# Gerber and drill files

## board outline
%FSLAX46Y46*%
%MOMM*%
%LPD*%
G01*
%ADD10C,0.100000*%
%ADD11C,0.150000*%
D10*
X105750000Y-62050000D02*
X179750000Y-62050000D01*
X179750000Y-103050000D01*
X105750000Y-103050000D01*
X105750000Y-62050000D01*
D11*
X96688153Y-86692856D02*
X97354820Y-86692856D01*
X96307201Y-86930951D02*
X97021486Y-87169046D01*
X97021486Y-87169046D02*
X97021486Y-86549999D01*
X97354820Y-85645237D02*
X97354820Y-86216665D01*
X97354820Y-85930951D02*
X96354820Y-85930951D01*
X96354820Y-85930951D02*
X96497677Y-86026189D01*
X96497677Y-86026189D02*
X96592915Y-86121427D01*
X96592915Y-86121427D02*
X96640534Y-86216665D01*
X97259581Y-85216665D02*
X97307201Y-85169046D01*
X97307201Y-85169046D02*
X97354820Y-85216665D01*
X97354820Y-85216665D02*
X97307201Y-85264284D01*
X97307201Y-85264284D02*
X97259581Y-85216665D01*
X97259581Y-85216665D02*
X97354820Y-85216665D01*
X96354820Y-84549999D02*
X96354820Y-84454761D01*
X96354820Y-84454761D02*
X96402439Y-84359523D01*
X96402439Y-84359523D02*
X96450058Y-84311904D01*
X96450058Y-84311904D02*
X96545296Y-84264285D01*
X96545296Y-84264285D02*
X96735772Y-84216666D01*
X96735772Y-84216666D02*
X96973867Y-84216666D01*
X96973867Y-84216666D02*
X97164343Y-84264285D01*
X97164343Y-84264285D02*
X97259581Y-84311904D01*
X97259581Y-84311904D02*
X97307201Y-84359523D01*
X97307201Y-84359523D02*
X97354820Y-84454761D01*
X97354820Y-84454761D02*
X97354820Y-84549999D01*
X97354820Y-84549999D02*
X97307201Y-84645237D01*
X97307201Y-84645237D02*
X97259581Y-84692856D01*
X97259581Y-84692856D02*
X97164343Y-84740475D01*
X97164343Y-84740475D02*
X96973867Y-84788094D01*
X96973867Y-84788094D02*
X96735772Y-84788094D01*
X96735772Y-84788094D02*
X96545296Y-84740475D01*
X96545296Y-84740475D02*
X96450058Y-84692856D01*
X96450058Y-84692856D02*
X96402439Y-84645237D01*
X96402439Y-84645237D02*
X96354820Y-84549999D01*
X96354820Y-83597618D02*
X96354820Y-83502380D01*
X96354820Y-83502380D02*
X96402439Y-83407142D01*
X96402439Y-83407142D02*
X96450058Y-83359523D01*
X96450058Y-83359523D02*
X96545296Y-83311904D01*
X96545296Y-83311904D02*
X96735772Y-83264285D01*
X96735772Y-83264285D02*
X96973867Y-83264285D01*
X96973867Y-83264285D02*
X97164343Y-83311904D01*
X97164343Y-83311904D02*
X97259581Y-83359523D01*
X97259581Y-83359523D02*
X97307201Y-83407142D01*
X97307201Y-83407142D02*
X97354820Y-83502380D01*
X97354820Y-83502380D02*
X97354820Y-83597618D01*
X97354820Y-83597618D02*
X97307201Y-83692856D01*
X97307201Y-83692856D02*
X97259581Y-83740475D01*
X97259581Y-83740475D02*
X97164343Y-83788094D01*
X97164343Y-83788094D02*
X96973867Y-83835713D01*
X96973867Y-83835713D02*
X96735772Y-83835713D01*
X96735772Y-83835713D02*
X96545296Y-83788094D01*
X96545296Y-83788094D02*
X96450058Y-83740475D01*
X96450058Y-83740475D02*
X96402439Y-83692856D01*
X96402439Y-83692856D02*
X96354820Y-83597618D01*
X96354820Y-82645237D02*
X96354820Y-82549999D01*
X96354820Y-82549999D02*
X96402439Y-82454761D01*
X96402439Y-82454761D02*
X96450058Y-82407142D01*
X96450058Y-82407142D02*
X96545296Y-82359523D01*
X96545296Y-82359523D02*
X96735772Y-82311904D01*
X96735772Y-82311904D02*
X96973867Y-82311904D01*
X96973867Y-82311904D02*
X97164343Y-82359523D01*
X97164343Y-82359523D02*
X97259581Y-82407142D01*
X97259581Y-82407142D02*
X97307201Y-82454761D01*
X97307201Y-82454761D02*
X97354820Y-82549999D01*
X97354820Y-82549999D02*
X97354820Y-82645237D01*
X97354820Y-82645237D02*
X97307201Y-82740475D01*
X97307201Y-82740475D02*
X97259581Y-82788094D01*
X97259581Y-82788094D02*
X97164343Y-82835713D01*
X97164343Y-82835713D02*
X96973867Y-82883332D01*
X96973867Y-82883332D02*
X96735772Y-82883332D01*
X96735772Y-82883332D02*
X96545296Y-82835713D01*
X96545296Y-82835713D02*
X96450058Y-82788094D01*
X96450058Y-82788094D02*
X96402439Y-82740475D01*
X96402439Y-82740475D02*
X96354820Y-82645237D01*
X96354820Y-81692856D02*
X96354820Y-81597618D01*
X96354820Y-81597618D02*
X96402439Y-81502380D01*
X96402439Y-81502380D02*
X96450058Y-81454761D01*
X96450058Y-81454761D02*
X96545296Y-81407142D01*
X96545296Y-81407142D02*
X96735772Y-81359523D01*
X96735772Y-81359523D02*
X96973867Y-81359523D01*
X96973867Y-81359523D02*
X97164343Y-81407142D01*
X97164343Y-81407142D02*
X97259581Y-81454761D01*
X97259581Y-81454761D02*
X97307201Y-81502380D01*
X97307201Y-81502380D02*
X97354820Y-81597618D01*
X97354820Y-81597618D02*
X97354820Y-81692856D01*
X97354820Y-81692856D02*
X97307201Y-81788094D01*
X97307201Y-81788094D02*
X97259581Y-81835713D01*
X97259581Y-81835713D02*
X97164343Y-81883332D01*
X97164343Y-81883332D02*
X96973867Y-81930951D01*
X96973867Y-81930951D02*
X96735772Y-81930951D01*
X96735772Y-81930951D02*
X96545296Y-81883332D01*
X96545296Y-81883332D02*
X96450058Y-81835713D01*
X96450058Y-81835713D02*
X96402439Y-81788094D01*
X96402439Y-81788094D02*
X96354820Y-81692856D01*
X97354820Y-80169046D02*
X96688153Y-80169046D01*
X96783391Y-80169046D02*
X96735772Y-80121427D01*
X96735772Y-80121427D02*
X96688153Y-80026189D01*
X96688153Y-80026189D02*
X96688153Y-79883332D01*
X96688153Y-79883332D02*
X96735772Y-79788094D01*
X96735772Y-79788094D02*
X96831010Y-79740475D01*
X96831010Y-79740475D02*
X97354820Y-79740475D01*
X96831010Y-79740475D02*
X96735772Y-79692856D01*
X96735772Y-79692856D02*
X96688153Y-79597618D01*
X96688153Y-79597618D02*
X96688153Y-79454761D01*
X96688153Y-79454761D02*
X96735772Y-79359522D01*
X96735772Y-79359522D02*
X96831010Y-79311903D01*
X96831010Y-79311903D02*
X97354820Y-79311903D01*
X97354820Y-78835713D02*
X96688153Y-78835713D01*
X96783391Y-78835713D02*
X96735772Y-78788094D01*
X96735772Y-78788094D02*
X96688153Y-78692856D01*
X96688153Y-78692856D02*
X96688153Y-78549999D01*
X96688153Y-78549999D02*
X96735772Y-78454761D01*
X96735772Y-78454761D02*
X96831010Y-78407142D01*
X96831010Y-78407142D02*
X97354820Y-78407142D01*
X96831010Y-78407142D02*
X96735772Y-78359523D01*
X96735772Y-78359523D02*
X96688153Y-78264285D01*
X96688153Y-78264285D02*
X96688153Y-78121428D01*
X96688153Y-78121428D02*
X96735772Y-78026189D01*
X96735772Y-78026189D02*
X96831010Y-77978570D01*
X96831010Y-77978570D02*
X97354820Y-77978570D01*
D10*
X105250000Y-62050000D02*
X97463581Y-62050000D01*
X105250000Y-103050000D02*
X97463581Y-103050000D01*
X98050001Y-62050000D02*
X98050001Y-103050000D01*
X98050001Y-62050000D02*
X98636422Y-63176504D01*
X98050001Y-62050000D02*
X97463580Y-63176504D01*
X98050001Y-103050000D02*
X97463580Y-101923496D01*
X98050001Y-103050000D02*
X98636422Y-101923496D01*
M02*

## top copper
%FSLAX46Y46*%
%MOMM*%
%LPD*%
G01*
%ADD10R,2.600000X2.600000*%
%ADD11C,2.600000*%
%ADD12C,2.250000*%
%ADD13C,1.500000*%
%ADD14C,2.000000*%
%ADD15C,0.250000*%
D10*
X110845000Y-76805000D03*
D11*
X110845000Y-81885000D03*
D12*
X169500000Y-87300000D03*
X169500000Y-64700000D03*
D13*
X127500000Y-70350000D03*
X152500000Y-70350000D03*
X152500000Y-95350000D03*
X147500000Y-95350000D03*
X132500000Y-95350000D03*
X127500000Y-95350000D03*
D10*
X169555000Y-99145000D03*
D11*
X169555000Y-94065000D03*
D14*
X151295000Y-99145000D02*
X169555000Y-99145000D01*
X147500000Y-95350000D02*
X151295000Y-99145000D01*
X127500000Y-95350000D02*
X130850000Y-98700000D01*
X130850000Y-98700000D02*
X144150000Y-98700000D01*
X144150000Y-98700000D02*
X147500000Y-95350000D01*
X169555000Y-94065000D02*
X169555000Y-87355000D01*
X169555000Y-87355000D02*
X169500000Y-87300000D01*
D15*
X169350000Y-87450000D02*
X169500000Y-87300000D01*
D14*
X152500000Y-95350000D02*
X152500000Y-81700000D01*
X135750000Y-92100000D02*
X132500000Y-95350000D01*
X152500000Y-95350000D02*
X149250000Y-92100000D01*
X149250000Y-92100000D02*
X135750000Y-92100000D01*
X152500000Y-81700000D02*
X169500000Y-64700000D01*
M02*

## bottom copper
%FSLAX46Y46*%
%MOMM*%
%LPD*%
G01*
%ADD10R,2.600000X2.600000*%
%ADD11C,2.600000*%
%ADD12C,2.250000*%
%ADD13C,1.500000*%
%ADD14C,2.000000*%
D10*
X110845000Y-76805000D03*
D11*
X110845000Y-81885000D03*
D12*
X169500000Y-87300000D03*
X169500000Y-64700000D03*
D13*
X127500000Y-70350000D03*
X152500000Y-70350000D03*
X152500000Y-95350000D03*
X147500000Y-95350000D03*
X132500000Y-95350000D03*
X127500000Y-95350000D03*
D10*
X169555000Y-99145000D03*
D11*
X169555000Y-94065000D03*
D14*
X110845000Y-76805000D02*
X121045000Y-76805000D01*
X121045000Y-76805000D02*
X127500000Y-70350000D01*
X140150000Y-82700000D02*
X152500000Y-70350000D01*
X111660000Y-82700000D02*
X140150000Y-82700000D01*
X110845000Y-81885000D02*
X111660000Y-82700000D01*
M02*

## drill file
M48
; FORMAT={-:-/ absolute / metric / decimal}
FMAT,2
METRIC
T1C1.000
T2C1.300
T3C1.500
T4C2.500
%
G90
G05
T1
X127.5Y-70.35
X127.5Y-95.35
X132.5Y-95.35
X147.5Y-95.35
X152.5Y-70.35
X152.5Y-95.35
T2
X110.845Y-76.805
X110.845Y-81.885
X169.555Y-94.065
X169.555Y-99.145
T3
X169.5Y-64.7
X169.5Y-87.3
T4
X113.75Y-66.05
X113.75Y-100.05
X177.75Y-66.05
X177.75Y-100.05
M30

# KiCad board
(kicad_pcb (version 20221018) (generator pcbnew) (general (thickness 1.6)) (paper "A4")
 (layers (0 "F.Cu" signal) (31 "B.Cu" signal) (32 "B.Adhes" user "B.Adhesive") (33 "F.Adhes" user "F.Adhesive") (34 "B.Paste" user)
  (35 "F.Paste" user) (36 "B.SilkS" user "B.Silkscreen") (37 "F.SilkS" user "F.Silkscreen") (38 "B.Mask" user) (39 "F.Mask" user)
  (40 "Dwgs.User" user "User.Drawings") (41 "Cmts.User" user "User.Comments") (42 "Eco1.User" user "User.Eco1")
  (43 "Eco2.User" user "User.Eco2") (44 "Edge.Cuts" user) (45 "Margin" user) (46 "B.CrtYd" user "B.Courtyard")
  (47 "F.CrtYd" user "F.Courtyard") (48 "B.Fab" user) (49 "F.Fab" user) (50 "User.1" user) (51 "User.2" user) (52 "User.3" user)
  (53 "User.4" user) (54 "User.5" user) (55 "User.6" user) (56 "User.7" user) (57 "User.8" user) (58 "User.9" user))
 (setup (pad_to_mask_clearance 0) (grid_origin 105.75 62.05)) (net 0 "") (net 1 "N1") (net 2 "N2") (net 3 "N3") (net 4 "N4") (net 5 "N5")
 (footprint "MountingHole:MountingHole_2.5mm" (layer "F.Cu") (at 113.75 100.05)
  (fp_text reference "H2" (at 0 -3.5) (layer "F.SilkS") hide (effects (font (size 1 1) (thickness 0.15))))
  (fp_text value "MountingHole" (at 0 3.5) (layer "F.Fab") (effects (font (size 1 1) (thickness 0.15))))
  (pad "" np_thru_hole circle (at 0 0) (size 2.5 2.5) (drill 2.5) (layers "*.Cu" "*.Mask")))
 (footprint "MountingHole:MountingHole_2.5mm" (layer "F.Cu") (at 113.75 66.05)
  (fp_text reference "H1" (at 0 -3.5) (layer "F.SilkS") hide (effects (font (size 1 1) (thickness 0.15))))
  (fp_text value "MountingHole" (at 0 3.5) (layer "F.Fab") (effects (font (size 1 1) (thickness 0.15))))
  (pad "" np_thru_hole circle (at 0 0) (size 2.5 2.5) (drill 2.5) (layers "*.Cu" "*.Mask")))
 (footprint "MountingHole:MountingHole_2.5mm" (layer "F.Cu") (at 177.75 100.05)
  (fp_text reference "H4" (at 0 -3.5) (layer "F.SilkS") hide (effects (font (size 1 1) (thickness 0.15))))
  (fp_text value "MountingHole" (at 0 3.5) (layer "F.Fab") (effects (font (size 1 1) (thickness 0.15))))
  (pad "" np_thru_hole circle (at 0 0) (size 2.5 2.5) (drill 2.5) (layers "*.Cu" "*.Mask")))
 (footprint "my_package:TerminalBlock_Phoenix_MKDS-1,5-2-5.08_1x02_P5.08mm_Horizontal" (layer "F.Cu") (at 110.845 76.805 -90)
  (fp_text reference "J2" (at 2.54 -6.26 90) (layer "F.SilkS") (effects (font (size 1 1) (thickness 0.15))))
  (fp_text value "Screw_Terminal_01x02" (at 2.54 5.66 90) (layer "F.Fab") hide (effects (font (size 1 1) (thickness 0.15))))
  (pad "1" thru_hole rect (at 0 0 270) (size 2.6 2.6) (drill 1.3) (layers "*.Cu" "*.Mask") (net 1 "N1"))
  (pad "2" thru_hole circle (at 5.08 0 270) (size 2.6 2.6) (drill 1.3) (layers "*.Cu" "*.Mask") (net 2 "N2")))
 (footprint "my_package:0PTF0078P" (layer "F.Cu") (at 169.5 76 90)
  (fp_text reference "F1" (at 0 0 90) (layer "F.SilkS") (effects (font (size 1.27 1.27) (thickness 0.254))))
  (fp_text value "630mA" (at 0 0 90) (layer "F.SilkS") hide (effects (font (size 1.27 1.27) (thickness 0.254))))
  (pad "1" thru_hole circle (at -11.3 0 90) (size 2.25 2.25) (drill 1.5) (layers "*.Cu" "*.Mask") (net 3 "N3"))
  (pad "2" thru_hole circle (at 11.3 0 90) (size 2.25 2.25) (drill 1.5) (layers "*.Cu" "*.Mask") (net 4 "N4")))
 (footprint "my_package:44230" (layer "F.Cu") (at 127.5 70.35)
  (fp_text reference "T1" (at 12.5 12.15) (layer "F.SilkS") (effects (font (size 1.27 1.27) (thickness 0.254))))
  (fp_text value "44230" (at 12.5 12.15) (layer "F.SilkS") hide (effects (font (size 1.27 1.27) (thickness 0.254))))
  (pad "1" thru_hole circle (at 0 0) (size 1.5 1.5) (drill 1) (layers "*.Cu" "*.Mask") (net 1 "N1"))
  (pad "5" thru_hole circle (at 25 0) (size 1.5 1.5) (drill 1) (layers "*.Cu" "*.Mask") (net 2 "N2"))
  (pad "6" thru_hole circle (at 25 25) (size 1.5 1.5) (drill 1) (layers "*.Cu" "*.Mask") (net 4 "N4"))
  (pad "7" thru_hole circle (at 20 25) (size 1.5 1.5) (drill 1) (layers "*.Cu" "*.Mask") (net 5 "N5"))
  (pad "9" thru_hole circle (at 5 25) (size 1.5 1.5) (drill 1) (layers "*.Cu" "*.Mask") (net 4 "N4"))
  (pad "10" thru_hole circle (at 0 25) (size 1.5 1.5) (drill 1) (layers "*.Cu" "*.Mask") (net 5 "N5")))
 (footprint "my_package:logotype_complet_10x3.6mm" (layer "F.Cu") (at 111.4 70.95)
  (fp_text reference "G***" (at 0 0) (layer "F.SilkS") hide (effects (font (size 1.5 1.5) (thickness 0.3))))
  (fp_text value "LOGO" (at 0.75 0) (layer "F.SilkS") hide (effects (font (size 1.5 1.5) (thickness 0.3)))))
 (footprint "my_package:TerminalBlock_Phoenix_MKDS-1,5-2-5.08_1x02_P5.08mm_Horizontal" (layer "F.Cu") (at 169.555 99.145 90)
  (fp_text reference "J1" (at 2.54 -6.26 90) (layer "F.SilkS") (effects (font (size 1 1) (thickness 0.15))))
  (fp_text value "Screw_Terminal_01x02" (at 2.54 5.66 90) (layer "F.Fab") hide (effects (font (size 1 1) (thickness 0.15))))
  (pad "1" thru_hole rect (at 0 0 90) (size 2.6 2.6) (drill 1.3) (layers "*.Cu" "*.Mask") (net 5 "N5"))
  (pad "2" thru_hole circle (at 5.08 0 90) (size 2.6 2.6) (drill 1.3) (layers "*.Cu" "*.Mask") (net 3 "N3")))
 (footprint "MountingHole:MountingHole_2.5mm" (layer "F.Cu") (at 177.75 66.05)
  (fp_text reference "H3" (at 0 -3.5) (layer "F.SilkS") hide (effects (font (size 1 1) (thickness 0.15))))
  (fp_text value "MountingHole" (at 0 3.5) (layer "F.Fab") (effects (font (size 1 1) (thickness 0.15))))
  (pad "" np_thru_hole circle (at 0 0) (size 2.5 2.5) (drill 2.5) (layers "*.Cu" "*.Mask")))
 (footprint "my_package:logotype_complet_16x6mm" (layer "B.Cu") (at 142.75 67.05 180)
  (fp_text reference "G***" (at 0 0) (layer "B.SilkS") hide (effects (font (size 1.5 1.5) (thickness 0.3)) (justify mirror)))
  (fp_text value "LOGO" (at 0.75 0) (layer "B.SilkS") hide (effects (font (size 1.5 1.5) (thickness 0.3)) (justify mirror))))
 (gr_rect locked (start 105.75 62.05) (end 179.75 103.05) (stroke (width 0.1) (type default)) (fill none) (layer "Edge.Cuts"))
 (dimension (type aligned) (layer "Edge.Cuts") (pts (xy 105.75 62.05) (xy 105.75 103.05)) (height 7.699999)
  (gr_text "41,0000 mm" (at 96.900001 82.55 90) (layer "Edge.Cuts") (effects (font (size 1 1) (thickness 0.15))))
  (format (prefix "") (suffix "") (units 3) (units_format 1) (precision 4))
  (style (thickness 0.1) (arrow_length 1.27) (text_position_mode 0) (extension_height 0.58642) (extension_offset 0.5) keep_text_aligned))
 (segment (start 151.295 99.145) (end 169.555 99.145) (width 2) (layer "F.Cu") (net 5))
 (segment (start 147.5 95.35) (end 151.295 99.145) (width 2) (layer "F.Cu") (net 5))
 (segment (start 127.5 95.35) (end 130.85 98.7) (width 2) (layer "F.Cu") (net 5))
 (segment (start 130.85 98.7) (end 144.15 98.7) (width 2) (layer "F.Cu") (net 5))
 (segment (start 144.15 98.7) (end 147.5 95.35) (width 2) (layer "F.Cu") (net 5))
 (segment (start 169.555 94.065) (end 169.555 87.355) (width 2) (layer "F.Cu") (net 3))
 (segment (start 169.555 87.355) (end 169.5 87.3) (width 2) (layer "F.Cu") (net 3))
 (segment (start 169.35 87.45) (end 169.5 87.3) (width 0.25) (layer "F.Cu") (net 3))
 (segment (start 110.845 76.805) (end 121.045 76.805) (width 2) (layer "B.Cu") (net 1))
 (segment (start 121.045 76.805) (end 127.5 70.35) (width 2) (layer "B.Cu") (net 1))
 (segment (start 140.15 82.7) (end 152.5 70.35) (width 2) (layer "B.Cu") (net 2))
 (segment (start 111.66 82.7) (end 140.15 82.7) (width 2) (layer "B.Cu") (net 2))
 (segment (start 110.845 81.885) (end 111.66 82.7) (width 2) (layer "B.Cu") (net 2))
 (segment (start 152.5 95.35) (end 152.5 81.7) (width 2) (layer "F.Cu") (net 4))
 (segment (start 135.75 92.1) (end 132.5 95.35) (width 2) (layer "F.Cu") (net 4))
 (segment (start 152.5 95.35) (end 149.25 92.1) (width 2) (layer "F.Cu") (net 4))
 (segment (start 149.25 92.1) (end 135.75 92.1) (width 2) (layer "F.Cu") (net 4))
 (segment (start 152.5 81.7) (end 169.5 64.7) (width 2) (layer "F.Cu") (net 4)))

